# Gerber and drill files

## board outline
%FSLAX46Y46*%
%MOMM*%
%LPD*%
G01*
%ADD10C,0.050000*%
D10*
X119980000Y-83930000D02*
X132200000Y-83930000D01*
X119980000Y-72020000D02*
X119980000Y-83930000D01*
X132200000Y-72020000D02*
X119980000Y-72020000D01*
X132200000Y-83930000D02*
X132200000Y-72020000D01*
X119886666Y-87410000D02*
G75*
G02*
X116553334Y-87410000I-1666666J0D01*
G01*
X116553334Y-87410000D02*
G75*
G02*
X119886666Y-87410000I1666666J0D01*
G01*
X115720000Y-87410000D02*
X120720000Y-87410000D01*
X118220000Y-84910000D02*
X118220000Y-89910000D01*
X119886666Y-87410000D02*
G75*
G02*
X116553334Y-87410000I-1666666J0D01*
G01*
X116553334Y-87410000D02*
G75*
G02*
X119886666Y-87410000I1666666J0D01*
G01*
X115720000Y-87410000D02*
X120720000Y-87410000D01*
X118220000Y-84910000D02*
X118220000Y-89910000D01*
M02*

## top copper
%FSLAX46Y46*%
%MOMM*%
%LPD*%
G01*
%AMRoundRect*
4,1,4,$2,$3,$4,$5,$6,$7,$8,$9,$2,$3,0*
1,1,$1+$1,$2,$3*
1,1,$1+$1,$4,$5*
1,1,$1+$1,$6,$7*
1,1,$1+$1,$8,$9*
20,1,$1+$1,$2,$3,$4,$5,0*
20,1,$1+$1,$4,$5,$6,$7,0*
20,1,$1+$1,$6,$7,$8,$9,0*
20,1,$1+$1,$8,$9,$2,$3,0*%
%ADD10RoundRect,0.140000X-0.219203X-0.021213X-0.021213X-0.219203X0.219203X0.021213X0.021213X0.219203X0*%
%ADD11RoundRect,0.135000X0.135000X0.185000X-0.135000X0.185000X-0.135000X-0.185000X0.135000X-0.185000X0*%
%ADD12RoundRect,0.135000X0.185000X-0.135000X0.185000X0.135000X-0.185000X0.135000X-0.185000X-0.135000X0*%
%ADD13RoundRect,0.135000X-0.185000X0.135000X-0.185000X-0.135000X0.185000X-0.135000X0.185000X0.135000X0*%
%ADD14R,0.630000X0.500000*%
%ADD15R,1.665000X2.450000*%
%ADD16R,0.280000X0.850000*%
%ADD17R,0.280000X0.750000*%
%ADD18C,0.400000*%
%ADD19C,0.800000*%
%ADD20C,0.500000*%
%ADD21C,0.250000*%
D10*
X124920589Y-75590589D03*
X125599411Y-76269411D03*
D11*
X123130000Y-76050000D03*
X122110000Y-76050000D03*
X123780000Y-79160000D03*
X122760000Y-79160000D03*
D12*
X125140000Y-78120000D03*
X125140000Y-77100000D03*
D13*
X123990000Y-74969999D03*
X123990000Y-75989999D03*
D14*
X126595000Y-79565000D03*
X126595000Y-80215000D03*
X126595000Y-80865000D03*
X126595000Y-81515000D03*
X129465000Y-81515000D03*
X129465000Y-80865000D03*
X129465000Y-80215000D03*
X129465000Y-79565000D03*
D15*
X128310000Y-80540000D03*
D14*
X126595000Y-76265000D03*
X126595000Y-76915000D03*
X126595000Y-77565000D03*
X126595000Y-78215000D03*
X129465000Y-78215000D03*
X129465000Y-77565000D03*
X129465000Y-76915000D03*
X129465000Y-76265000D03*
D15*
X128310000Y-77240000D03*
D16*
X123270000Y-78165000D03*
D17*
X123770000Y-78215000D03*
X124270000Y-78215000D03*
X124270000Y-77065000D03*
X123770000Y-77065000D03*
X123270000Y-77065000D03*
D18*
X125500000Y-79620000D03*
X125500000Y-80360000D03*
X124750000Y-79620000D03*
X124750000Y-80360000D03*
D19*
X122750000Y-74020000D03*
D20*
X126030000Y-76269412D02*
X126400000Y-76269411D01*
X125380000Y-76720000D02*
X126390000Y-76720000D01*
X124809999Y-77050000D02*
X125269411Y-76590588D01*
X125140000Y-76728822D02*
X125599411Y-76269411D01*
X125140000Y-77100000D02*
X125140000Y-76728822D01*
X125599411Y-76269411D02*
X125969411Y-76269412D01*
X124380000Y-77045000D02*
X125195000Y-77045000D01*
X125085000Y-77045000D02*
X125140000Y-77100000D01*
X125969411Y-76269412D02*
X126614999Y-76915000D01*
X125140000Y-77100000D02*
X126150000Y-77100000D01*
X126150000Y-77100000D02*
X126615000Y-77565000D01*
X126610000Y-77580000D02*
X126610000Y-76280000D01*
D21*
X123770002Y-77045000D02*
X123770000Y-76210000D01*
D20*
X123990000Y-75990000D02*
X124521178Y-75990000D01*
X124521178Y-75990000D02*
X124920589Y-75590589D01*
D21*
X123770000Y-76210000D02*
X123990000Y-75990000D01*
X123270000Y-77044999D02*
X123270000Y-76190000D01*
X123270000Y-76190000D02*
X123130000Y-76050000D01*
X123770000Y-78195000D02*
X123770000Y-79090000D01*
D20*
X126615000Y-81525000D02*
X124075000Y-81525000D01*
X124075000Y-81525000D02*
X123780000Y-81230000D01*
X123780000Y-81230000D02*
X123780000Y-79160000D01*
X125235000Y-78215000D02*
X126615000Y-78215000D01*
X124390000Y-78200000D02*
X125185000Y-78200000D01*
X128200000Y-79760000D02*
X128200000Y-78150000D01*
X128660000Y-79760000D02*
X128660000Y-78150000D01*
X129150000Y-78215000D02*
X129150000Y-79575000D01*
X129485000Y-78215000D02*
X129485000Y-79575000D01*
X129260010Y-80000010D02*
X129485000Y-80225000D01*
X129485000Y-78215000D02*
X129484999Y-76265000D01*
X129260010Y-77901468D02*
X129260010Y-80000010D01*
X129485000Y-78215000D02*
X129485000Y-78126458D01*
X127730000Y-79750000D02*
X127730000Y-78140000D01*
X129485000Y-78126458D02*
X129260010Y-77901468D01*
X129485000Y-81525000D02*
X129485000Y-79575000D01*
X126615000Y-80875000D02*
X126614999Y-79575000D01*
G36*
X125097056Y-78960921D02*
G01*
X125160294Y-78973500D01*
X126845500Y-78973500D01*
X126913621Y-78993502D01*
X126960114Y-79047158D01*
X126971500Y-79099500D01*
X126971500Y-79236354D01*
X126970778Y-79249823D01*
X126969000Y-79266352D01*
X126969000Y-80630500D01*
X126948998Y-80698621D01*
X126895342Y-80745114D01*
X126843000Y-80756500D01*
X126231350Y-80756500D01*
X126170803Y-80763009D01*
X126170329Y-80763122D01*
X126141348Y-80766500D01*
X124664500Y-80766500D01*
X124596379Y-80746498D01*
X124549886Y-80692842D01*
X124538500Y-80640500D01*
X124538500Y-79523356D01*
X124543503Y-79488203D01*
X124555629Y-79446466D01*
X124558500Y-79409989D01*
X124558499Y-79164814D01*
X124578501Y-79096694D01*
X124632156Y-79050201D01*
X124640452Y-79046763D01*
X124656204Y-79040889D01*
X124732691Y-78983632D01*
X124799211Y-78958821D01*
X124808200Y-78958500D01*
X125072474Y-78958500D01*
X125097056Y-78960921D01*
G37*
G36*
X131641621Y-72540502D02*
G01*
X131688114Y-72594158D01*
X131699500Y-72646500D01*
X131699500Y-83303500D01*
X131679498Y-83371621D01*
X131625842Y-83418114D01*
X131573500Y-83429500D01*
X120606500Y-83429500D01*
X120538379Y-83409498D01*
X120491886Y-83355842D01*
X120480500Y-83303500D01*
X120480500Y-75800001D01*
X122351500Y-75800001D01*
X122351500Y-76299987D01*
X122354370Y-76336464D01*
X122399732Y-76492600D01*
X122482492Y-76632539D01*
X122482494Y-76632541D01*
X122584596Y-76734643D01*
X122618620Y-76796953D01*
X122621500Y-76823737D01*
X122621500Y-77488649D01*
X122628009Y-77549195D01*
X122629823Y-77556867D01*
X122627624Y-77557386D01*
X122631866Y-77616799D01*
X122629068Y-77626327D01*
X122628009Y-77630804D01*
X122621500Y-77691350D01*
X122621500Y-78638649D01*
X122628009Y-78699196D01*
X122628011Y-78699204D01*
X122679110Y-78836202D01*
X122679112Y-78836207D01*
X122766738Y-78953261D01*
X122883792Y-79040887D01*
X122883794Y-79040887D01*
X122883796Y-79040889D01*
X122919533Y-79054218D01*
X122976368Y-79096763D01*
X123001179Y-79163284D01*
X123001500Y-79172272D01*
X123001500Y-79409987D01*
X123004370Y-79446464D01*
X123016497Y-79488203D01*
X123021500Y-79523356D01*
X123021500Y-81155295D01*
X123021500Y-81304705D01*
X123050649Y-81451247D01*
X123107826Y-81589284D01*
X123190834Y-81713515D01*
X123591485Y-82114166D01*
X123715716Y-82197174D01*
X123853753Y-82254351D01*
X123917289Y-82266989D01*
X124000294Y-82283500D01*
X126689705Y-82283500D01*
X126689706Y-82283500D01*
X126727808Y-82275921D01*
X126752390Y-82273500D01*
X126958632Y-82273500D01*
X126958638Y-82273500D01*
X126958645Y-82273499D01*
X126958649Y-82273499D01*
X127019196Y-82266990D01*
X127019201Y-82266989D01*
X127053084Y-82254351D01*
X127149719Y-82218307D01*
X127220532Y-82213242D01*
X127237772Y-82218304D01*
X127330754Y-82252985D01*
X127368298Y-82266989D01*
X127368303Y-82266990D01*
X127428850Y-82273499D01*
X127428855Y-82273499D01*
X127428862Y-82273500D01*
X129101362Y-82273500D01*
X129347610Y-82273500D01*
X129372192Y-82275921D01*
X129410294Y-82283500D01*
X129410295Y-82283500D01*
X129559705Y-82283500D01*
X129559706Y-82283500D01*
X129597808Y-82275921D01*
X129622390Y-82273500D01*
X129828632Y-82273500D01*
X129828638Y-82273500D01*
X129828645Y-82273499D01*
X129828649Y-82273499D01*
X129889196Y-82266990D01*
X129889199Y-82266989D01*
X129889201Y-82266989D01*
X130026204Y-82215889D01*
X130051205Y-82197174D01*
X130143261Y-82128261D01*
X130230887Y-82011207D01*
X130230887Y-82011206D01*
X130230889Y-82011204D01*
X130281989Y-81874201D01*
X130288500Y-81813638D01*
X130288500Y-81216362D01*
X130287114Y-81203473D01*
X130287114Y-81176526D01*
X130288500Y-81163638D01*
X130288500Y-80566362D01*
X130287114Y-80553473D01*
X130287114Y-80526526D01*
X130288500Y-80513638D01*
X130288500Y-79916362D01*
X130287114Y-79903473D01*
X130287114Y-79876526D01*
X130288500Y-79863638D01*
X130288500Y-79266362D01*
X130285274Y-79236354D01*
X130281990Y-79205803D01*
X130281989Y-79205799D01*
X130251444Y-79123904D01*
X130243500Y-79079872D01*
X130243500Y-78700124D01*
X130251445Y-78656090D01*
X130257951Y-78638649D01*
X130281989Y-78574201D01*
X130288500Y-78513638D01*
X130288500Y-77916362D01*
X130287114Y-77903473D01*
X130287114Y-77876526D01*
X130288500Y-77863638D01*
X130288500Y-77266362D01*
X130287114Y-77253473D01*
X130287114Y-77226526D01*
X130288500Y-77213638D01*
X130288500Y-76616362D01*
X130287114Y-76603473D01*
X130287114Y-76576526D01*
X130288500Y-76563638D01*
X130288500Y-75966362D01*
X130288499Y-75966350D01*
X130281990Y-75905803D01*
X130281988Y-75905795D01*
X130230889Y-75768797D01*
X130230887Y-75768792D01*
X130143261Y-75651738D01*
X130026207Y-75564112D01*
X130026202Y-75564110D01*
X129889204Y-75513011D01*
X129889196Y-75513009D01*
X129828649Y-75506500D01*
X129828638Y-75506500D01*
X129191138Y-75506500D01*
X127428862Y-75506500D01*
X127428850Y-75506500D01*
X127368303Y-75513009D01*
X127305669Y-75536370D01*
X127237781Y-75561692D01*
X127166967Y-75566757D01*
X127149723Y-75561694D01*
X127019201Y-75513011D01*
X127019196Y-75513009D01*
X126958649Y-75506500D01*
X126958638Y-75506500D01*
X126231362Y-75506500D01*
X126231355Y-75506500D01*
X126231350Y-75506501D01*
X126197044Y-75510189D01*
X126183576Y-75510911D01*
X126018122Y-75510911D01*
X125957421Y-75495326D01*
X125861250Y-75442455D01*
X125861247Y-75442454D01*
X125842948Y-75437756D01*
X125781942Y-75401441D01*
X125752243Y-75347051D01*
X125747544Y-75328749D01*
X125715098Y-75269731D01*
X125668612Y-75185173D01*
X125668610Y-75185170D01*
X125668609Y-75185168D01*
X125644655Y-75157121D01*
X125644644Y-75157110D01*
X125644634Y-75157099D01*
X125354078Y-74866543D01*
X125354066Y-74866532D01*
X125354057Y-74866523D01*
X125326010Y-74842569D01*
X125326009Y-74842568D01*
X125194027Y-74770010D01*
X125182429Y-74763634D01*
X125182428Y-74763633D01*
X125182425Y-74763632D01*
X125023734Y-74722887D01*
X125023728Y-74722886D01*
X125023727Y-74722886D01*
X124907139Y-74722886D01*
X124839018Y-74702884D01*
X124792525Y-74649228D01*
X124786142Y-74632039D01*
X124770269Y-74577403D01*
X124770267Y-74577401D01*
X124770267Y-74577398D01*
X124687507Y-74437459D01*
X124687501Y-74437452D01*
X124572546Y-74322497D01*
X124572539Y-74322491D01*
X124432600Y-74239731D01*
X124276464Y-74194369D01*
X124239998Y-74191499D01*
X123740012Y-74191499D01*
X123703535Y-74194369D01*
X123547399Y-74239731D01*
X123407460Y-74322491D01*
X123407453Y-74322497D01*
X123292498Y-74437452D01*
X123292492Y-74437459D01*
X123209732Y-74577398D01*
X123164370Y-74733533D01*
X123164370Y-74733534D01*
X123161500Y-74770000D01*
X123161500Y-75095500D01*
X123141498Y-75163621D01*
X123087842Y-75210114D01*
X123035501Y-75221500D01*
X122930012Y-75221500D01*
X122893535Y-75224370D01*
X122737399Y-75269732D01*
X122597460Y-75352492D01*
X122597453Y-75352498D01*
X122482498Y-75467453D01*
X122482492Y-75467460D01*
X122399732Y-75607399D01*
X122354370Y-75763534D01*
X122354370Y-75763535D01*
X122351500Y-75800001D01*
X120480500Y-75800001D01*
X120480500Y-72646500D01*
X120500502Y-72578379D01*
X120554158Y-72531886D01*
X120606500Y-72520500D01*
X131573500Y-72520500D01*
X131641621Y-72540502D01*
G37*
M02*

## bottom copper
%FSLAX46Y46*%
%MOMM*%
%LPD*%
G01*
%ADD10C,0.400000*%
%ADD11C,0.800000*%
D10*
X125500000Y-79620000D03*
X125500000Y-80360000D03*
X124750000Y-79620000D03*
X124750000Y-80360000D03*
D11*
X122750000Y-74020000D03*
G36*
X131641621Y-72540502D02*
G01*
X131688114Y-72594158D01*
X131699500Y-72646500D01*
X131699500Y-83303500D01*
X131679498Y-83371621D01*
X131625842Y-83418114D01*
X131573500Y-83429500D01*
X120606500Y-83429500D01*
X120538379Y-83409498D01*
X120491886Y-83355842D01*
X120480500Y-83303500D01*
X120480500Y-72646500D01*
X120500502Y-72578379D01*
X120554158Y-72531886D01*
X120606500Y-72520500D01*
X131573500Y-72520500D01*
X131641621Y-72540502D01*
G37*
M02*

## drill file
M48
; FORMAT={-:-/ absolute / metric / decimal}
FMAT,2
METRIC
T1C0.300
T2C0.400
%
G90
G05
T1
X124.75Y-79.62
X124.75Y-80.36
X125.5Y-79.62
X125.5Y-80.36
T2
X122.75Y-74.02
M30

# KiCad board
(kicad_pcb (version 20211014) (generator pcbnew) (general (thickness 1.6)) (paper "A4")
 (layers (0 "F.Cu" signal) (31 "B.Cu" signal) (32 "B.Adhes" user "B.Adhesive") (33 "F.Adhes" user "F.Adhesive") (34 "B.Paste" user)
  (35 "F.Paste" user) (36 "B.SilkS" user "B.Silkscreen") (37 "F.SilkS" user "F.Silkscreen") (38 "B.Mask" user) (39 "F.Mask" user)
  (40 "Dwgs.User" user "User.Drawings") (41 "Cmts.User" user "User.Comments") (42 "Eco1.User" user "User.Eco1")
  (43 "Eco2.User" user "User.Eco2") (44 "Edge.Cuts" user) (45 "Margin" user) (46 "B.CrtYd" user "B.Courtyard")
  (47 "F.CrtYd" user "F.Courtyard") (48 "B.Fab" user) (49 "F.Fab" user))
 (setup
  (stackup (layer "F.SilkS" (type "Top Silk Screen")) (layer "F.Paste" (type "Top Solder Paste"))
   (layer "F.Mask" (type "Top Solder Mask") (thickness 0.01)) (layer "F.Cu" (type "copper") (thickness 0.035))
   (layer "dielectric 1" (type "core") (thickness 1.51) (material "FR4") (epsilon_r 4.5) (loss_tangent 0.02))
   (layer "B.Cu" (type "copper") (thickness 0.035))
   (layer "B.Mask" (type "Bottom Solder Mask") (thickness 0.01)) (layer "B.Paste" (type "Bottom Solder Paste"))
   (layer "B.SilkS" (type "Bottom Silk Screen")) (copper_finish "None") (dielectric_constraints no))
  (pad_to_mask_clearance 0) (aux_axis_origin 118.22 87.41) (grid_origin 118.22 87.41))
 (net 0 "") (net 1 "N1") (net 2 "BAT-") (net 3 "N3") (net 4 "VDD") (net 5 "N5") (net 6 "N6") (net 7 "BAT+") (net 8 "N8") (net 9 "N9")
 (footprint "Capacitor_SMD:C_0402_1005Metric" (layer "F.Cu") (at 125.26 75.93 -45)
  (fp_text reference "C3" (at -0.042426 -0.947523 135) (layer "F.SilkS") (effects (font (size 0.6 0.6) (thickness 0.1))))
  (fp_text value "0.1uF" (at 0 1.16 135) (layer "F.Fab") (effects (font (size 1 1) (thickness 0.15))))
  (pad "1" smd roundrect locked (at -0.48 0 315) (size 0.56 0.62) (layers "F.Cu" "F.Paste" "F.Mask") (roundrect_rratio 0.25) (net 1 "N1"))
  (pad "2" smd roundrect locked (at 0.48 0 315) (size 0.56 0.62) (layers "F.Cu" "F.Paste" "F.Mask") (roundrect_rratio 0.25) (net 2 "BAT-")))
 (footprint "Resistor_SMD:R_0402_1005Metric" (layer "F.Cu") (at 122.62 76.05 180)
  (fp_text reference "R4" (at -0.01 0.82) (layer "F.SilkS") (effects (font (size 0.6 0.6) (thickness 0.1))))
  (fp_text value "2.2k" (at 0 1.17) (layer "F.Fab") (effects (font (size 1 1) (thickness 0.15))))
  (pad "1" smd roundrect locked (at -0.51 0 180) (size 0.54 0.64) (layers "F.Cu" "F.Paste" "F.Mask") (roundrect_rratio 0.25) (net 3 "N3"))
  (pad "2" smd roundrect locked (at 0.51 0 180) (size 0.54 0.64) (layers "F.Cu" "F.Paste" "F.Mask") (roundrect_rratio 0.25) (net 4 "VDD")))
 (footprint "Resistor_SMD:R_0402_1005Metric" (layer "F.Cu") (at 123.27 79.16 180)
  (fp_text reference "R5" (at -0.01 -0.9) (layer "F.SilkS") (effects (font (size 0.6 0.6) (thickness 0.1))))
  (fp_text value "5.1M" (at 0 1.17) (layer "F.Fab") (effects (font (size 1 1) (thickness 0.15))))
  (pad "1" smd roundrect locked (at -0.51 0 180) (size 0.54 0.64) (layers "F.Cu" "F.Paste" "F.Mask") (roundrect_rratio 0.25) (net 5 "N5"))
  (pad "2" smd roundrect locked (at 0.51 0 180) (size 0.54 0.64) (layers "F.Cu" "F.Paste" "F.Mask") (roundrect_rratio 0.25) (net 4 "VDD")))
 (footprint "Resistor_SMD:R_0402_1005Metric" (layer "F.Cu") (at 125.14 77.61 90)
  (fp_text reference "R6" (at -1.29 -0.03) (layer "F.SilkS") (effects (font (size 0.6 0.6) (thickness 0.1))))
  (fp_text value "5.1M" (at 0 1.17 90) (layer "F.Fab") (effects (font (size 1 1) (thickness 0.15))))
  (pad "1" smd roundrect locked (at -0.51 0 90) (size 0.54 0.64) (layers "F.Cu" "F.Paste" "F.Mask") (roundrect_rratio 0.25) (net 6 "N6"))
  (pad "2" smd roundrect locked (at 0.51 0 90) (size 0.54 0.64) (layers "F.Cu" "F.Paste" "F.Mask") (roundrect_rratio 0.25) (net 2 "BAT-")))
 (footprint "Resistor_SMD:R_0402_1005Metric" (layer "F.Cu") (at 123.99 75.479999 -90)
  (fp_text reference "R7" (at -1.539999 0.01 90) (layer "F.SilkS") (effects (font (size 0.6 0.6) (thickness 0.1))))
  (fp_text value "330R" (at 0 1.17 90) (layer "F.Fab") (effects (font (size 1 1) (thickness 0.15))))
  (pad "1" smd roundrect locked (at -0.51 0 270) (size 0.54 0.64) (layers "F.Cu" "F.Paste" "F.Mask") (roundrect_rratio 0.25) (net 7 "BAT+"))
  (pad "2" smd roundrect locked (at 0.51 0 270) (size 0.54 0.64) (layers "F.Cu" "F.Paste" "F.Mask") (roundrect_rratio 0.25) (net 1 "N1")))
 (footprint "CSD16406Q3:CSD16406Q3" (layer "F.Cu") (at 128.03 80.54)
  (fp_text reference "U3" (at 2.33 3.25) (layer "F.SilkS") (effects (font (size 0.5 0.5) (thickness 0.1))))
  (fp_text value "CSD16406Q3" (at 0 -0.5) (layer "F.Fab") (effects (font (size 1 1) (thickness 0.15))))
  (pad "1" smd rect (at -1.435 -0.975) (size 0.63 0.5) (layers "F.Cu" "F.Mask") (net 4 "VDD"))
  (pad "2" smd rect (at -1.435 -0.325) (size 0.63 0.5) (layers "F.Cu" "F.Mask") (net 4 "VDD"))
  (pad "3" smd rect (at -1.435 0.325) (size 0.63 0.5) (layers "F.Cu" "F.Mask") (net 4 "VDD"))
  (pad "4" smd rect (at -1.435 0.975) (size 0.63 0.5) (layers "F.Cu" "F.Mask") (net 5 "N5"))
  (pad "5" smd rect (at 1.435 0.975) (size 0.63 0.5) (layers "F.Cu") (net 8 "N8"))
  (pad "6" smd rect (at 1.435 0.325) (size 0.63 0.5) (layers "F.Cu") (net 8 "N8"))
  (pad "7" smd rect (at 1.435 -0.325) (size 0.63 0.5) (layers "F.Cu") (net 8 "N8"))
  (pad "8" smd rect (at 1.435 -0.975) (size 0.63 0.5) (layers "F.Cu") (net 8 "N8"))
  (pad "8" smd rect (at 0.28 0) (size 1.665 2.45) (layers "F.Cu") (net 8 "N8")))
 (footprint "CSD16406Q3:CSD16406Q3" (layer "F.Cu") (at 128.03 77.24)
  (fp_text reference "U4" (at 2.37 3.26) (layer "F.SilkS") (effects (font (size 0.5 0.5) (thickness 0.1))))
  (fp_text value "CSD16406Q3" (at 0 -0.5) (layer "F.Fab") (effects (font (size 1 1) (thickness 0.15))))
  (pad "1" smd rect (at -1.435 -0.975) (size 0.63 0.5) (layers "F.Cu" "F.Mask") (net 2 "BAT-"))
  (pad "2" smd rect (at -1.435 -0.325) (size 0.63 0.5) (layers "F.Cu" "F.Mask") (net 2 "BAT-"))
  (pad "3" smd rect (at -1.435 0.325) (size 0.63 0.5) (layers "F.Cu" "F.Mask") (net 2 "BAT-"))
  (pad "4" smd rect (at -1.435 0.975) (size 0.63 0.5) (layers "F.Cu" "F.Mask") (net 6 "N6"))
  (pad "5" smd rect (at 1.435 0.975) (size 0.63 0.5) (layers "F.Cu") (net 8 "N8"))
  (pad "6" smd rect (at 1.435 0.325) (size 0.63 0.5) (layers "F.Cu") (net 8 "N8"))
  (pad "7" smd rect (at 1.435 -0.325) (size 0.63 0.5) (layers "F.Cu") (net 8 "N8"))
  (pad "8" smd rect (at 1.435 -0.975) (size 0.63 0.5) (layers "F.Cu") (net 8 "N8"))
  (pad "8" smd rect (at 0.28 0) (size 1.665 2.45) (layers "F.Cu") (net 8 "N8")))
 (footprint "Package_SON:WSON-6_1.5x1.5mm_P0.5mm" (layer "F.Cu") (at 123.77 77.64 90)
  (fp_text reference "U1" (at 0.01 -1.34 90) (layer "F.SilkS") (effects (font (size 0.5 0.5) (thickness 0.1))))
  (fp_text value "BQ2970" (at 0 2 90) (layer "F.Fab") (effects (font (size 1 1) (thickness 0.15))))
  (pad "1" smd rect locked (at -0.525 -0.5) (size 0.28 0.85) (layers "F.Cu" "F.Paste" "F.Mask") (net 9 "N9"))
  (pad "2" smd rect locked (at -0.575 0) (size 0.28 0.75) (layers "F.Cu" "F.Paste" "F.Mask") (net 5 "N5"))
  (pad "3" smd rect locked (at -0.575 0.5) (size 0.28 0.75) (layers "F.Cu" "F.Paste" "F.Mask") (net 6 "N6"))
  (pad "4" smd rect locked (at 0.575 0.5) (size 0.28 0.75) (layers "F.Cu" "F.Paste" "F.Mask") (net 2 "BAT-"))
  (pad "5" smd rect locked (at 0.575 0) (size 0.28 0.75) (layers "F.Cu" "F.Paste" "F.Mask") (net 1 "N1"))
  (pad "6" smd rect locked (at 0.575 -0.5) (size 0.28 0.75) (layers "F.Cu" "F.Paste" "F.Mask") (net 3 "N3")))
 (gr_line (start 119.98 83.93) (end 132.2 83.93) (layer "Edge.Cuts") (width 0.05))
 (gr_line (start 119.98 72.02) (end 119.98 83.93) (layer "Edge.Cuts") (width 0.05))
 (gr_line (start 132.2 72.02) (end 119.98 72.02) (layer "Edge.Cuts") (width 0.05))
 (gr_line (start 132.2 83.93) (end 132.2 72.02) (layer "Edge.Cuts") (width 0.05))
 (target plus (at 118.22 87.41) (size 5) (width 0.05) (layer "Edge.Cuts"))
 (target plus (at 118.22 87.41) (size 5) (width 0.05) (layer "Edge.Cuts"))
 (segment (start 126.03 76.269412) (end 126.4 76.269411) (width 0.5) (layer "F.Cu") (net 2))
 (segment (start 125.38 76.72) (end 126.39 76.72) (width 0.5) (layer "F.Cu") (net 2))
 (segment (start 124.809999 77.05) (end 125.269411 76.590588) (width 0.5) (layer "F.Cu") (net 2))
 (segment (start 125.14 76.728822) (end 125.599411 76.269411) (width 0.5) (layer "F.Cu") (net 2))
 (segment (start 125.14 77.1) (end 125.14 76.728822) (width 0.5) (layer "F.Cu") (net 2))
 (segment (start 125.599411 76.269411) (end 125.969411 76.269412) (width 0.5) (layer "F.Cu") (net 2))
 (segment (start 124.38 77.045) (end 125.195 77.045) (width 0.5) (layer "F.Cu") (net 2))
 (segment (start 125.085 77.045) (end 125.14 77.1) (width 0.5) (layer "F.Cu") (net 2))
 (segment (start 125.969411 76.269412) (end 126.614999 76.915) (width 0.5) (layer "F.Cu") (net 2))
 (segment (start 125.14 77.1) (end 126.15 77.1) (width 0.5) (layer "F.Cu") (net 2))
 (segment (start 126.15 77.1) (end 126.615 77.565) (width 0.5) (layer "F.Cu") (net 2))
 (segment (start 126.61 77.58) (end 126.61 76.28) (width 0.5) (layer "F.Cu") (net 2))
 (segment (start 123.770002 77.045) (end 123.77 76.21) (width 0.25) (layer "F.Cu") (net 1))
 (segment (start 123.99 75.99) (end 124.521178 75.99) (width 0.5) (layer "F.Cu") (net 1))
 (segment (start 124.521178 75.99) (end 124.920589 75.590589) (width 0.5) (layer "F.Cu") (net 1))
 (segment (start 123.77 76.21) (end 123.99 75.99) (width 0.25) (layer "F.Cu") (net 1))
 (segment (start 123.27 77.044999) (end 123.27 76.19) (width 0.25) (layer "F.Cu") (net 3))
 (segment (start 123.27 76.19) (end 123.13 76.05) (width 0.25) (layer "F.Cu") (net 3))
 (segment (start 123.77 78.195) (end 123.77 79.09) (width 0.25) (layer "F.Cu") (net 5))
 (segment (start 126.615 81.525) (end 124.075 81.525) (width 0.5) (layer "F.Cu") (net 5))
 (segment (start 124.075 81.525) (end 123.78 81.23) (width 0.5) (layer "F.Cu") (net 5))
 (segment (start 123.78 81.23) (end 123.78 79.16) (width 0.5) (layer "F.Cu") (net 5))
 (segment (start 125.235 78.215) (end 126.615 78.215) (width 0.5) (layer "F.Cu") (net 6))
 (segment (start 124.39 78.2) (end 125.185 78.2) (width 0.5) (layer "F.Cu") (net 6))
 (segment (start 128.2 79.76) (end 128.2 78.15) (width 0.5) (layer "F.Cu") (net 8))
 (segment (start 128.66 79.76) (end 128.66 78.15) (width 0.5) (layer "F.Cu") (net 8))
 (segment (start 129.15 78.215) (end 129.15 79.575) (width 0.5) (layer "F.Cu") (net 8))
 (segment (start 129.485 78.215) (end 129.485 79.575) (width 0.5) (layer "F.Cu") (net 8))
 (segment (start 129.26001 80.00001) (end 129.485 80.225) (width 0.5) (layer "F.Cu") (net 8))
 (segment (start 129.485 78.215) (end 129.484999 76.265) (width 0.5) (layer "F.Cu") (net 8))
 (segment (start 129.26001 77.901468) (end 129.26001 80.00001) (width 0.5) (layer "F.Cu") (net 8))
 (segment (start 129.485 78.215) (end 129.485 78.126458) (width 0.5) (layer "F.Cu") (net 8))
 (segment (start 127.73 79.75) (end 127.73 78.14) (width 0.5) (layer "F.Cu") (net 8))
 (segment (start 129.485 78.126458) (end 129.26001 77.901468) (width 0.5) (layer "F.Cu") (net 8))
 (segment (start 129.485 81.525) (end 129.485 79.575) (width 0.5) (layer "F.Cu") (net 8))
 (segment (start 126.615 80.875) (end 126.614999 79.575) (width 0.5) (layer "F.Cu") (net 4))
 (via (at 125.5 79.62) (size 0.4) (drill 0.3) (layers "F.Cu" "B.Cu") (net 4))
 (via (at 125.5 80.36) (size 0.4) (drill 0.3) (layers "F.Cu" "B.Cu") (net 4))
 (via (at 124.75 79.62) (size 0.4) (drill 0.3) (layers "F.Cu" "B.Cu") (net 4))
 (via (at 124.75 80.36) (size 0.4) (drill 0.3) (layers "F.Cu" "B.Cu") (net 4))
 (via (at 122.75 74.02) (size 0.8) (drill 0.4) (layers "F.Cu" "B.Cu") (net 4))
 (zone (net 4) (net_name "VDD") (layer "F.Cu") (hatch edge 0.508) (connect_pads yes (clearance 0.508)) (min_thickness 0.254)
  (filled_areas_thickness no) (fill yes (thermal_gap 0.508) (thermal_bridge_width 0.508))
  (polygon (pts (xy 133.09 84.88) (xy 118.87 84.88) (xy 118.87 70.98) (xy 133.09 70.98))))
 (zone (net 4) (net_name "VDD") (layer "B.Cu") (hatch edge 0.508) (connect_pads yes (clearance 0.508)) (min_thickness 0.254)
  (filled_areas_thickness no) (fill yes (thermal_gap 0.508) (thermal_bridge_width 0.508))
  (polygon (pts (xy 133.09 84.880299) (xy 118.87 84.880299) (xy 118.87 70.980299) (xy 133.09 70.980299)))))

